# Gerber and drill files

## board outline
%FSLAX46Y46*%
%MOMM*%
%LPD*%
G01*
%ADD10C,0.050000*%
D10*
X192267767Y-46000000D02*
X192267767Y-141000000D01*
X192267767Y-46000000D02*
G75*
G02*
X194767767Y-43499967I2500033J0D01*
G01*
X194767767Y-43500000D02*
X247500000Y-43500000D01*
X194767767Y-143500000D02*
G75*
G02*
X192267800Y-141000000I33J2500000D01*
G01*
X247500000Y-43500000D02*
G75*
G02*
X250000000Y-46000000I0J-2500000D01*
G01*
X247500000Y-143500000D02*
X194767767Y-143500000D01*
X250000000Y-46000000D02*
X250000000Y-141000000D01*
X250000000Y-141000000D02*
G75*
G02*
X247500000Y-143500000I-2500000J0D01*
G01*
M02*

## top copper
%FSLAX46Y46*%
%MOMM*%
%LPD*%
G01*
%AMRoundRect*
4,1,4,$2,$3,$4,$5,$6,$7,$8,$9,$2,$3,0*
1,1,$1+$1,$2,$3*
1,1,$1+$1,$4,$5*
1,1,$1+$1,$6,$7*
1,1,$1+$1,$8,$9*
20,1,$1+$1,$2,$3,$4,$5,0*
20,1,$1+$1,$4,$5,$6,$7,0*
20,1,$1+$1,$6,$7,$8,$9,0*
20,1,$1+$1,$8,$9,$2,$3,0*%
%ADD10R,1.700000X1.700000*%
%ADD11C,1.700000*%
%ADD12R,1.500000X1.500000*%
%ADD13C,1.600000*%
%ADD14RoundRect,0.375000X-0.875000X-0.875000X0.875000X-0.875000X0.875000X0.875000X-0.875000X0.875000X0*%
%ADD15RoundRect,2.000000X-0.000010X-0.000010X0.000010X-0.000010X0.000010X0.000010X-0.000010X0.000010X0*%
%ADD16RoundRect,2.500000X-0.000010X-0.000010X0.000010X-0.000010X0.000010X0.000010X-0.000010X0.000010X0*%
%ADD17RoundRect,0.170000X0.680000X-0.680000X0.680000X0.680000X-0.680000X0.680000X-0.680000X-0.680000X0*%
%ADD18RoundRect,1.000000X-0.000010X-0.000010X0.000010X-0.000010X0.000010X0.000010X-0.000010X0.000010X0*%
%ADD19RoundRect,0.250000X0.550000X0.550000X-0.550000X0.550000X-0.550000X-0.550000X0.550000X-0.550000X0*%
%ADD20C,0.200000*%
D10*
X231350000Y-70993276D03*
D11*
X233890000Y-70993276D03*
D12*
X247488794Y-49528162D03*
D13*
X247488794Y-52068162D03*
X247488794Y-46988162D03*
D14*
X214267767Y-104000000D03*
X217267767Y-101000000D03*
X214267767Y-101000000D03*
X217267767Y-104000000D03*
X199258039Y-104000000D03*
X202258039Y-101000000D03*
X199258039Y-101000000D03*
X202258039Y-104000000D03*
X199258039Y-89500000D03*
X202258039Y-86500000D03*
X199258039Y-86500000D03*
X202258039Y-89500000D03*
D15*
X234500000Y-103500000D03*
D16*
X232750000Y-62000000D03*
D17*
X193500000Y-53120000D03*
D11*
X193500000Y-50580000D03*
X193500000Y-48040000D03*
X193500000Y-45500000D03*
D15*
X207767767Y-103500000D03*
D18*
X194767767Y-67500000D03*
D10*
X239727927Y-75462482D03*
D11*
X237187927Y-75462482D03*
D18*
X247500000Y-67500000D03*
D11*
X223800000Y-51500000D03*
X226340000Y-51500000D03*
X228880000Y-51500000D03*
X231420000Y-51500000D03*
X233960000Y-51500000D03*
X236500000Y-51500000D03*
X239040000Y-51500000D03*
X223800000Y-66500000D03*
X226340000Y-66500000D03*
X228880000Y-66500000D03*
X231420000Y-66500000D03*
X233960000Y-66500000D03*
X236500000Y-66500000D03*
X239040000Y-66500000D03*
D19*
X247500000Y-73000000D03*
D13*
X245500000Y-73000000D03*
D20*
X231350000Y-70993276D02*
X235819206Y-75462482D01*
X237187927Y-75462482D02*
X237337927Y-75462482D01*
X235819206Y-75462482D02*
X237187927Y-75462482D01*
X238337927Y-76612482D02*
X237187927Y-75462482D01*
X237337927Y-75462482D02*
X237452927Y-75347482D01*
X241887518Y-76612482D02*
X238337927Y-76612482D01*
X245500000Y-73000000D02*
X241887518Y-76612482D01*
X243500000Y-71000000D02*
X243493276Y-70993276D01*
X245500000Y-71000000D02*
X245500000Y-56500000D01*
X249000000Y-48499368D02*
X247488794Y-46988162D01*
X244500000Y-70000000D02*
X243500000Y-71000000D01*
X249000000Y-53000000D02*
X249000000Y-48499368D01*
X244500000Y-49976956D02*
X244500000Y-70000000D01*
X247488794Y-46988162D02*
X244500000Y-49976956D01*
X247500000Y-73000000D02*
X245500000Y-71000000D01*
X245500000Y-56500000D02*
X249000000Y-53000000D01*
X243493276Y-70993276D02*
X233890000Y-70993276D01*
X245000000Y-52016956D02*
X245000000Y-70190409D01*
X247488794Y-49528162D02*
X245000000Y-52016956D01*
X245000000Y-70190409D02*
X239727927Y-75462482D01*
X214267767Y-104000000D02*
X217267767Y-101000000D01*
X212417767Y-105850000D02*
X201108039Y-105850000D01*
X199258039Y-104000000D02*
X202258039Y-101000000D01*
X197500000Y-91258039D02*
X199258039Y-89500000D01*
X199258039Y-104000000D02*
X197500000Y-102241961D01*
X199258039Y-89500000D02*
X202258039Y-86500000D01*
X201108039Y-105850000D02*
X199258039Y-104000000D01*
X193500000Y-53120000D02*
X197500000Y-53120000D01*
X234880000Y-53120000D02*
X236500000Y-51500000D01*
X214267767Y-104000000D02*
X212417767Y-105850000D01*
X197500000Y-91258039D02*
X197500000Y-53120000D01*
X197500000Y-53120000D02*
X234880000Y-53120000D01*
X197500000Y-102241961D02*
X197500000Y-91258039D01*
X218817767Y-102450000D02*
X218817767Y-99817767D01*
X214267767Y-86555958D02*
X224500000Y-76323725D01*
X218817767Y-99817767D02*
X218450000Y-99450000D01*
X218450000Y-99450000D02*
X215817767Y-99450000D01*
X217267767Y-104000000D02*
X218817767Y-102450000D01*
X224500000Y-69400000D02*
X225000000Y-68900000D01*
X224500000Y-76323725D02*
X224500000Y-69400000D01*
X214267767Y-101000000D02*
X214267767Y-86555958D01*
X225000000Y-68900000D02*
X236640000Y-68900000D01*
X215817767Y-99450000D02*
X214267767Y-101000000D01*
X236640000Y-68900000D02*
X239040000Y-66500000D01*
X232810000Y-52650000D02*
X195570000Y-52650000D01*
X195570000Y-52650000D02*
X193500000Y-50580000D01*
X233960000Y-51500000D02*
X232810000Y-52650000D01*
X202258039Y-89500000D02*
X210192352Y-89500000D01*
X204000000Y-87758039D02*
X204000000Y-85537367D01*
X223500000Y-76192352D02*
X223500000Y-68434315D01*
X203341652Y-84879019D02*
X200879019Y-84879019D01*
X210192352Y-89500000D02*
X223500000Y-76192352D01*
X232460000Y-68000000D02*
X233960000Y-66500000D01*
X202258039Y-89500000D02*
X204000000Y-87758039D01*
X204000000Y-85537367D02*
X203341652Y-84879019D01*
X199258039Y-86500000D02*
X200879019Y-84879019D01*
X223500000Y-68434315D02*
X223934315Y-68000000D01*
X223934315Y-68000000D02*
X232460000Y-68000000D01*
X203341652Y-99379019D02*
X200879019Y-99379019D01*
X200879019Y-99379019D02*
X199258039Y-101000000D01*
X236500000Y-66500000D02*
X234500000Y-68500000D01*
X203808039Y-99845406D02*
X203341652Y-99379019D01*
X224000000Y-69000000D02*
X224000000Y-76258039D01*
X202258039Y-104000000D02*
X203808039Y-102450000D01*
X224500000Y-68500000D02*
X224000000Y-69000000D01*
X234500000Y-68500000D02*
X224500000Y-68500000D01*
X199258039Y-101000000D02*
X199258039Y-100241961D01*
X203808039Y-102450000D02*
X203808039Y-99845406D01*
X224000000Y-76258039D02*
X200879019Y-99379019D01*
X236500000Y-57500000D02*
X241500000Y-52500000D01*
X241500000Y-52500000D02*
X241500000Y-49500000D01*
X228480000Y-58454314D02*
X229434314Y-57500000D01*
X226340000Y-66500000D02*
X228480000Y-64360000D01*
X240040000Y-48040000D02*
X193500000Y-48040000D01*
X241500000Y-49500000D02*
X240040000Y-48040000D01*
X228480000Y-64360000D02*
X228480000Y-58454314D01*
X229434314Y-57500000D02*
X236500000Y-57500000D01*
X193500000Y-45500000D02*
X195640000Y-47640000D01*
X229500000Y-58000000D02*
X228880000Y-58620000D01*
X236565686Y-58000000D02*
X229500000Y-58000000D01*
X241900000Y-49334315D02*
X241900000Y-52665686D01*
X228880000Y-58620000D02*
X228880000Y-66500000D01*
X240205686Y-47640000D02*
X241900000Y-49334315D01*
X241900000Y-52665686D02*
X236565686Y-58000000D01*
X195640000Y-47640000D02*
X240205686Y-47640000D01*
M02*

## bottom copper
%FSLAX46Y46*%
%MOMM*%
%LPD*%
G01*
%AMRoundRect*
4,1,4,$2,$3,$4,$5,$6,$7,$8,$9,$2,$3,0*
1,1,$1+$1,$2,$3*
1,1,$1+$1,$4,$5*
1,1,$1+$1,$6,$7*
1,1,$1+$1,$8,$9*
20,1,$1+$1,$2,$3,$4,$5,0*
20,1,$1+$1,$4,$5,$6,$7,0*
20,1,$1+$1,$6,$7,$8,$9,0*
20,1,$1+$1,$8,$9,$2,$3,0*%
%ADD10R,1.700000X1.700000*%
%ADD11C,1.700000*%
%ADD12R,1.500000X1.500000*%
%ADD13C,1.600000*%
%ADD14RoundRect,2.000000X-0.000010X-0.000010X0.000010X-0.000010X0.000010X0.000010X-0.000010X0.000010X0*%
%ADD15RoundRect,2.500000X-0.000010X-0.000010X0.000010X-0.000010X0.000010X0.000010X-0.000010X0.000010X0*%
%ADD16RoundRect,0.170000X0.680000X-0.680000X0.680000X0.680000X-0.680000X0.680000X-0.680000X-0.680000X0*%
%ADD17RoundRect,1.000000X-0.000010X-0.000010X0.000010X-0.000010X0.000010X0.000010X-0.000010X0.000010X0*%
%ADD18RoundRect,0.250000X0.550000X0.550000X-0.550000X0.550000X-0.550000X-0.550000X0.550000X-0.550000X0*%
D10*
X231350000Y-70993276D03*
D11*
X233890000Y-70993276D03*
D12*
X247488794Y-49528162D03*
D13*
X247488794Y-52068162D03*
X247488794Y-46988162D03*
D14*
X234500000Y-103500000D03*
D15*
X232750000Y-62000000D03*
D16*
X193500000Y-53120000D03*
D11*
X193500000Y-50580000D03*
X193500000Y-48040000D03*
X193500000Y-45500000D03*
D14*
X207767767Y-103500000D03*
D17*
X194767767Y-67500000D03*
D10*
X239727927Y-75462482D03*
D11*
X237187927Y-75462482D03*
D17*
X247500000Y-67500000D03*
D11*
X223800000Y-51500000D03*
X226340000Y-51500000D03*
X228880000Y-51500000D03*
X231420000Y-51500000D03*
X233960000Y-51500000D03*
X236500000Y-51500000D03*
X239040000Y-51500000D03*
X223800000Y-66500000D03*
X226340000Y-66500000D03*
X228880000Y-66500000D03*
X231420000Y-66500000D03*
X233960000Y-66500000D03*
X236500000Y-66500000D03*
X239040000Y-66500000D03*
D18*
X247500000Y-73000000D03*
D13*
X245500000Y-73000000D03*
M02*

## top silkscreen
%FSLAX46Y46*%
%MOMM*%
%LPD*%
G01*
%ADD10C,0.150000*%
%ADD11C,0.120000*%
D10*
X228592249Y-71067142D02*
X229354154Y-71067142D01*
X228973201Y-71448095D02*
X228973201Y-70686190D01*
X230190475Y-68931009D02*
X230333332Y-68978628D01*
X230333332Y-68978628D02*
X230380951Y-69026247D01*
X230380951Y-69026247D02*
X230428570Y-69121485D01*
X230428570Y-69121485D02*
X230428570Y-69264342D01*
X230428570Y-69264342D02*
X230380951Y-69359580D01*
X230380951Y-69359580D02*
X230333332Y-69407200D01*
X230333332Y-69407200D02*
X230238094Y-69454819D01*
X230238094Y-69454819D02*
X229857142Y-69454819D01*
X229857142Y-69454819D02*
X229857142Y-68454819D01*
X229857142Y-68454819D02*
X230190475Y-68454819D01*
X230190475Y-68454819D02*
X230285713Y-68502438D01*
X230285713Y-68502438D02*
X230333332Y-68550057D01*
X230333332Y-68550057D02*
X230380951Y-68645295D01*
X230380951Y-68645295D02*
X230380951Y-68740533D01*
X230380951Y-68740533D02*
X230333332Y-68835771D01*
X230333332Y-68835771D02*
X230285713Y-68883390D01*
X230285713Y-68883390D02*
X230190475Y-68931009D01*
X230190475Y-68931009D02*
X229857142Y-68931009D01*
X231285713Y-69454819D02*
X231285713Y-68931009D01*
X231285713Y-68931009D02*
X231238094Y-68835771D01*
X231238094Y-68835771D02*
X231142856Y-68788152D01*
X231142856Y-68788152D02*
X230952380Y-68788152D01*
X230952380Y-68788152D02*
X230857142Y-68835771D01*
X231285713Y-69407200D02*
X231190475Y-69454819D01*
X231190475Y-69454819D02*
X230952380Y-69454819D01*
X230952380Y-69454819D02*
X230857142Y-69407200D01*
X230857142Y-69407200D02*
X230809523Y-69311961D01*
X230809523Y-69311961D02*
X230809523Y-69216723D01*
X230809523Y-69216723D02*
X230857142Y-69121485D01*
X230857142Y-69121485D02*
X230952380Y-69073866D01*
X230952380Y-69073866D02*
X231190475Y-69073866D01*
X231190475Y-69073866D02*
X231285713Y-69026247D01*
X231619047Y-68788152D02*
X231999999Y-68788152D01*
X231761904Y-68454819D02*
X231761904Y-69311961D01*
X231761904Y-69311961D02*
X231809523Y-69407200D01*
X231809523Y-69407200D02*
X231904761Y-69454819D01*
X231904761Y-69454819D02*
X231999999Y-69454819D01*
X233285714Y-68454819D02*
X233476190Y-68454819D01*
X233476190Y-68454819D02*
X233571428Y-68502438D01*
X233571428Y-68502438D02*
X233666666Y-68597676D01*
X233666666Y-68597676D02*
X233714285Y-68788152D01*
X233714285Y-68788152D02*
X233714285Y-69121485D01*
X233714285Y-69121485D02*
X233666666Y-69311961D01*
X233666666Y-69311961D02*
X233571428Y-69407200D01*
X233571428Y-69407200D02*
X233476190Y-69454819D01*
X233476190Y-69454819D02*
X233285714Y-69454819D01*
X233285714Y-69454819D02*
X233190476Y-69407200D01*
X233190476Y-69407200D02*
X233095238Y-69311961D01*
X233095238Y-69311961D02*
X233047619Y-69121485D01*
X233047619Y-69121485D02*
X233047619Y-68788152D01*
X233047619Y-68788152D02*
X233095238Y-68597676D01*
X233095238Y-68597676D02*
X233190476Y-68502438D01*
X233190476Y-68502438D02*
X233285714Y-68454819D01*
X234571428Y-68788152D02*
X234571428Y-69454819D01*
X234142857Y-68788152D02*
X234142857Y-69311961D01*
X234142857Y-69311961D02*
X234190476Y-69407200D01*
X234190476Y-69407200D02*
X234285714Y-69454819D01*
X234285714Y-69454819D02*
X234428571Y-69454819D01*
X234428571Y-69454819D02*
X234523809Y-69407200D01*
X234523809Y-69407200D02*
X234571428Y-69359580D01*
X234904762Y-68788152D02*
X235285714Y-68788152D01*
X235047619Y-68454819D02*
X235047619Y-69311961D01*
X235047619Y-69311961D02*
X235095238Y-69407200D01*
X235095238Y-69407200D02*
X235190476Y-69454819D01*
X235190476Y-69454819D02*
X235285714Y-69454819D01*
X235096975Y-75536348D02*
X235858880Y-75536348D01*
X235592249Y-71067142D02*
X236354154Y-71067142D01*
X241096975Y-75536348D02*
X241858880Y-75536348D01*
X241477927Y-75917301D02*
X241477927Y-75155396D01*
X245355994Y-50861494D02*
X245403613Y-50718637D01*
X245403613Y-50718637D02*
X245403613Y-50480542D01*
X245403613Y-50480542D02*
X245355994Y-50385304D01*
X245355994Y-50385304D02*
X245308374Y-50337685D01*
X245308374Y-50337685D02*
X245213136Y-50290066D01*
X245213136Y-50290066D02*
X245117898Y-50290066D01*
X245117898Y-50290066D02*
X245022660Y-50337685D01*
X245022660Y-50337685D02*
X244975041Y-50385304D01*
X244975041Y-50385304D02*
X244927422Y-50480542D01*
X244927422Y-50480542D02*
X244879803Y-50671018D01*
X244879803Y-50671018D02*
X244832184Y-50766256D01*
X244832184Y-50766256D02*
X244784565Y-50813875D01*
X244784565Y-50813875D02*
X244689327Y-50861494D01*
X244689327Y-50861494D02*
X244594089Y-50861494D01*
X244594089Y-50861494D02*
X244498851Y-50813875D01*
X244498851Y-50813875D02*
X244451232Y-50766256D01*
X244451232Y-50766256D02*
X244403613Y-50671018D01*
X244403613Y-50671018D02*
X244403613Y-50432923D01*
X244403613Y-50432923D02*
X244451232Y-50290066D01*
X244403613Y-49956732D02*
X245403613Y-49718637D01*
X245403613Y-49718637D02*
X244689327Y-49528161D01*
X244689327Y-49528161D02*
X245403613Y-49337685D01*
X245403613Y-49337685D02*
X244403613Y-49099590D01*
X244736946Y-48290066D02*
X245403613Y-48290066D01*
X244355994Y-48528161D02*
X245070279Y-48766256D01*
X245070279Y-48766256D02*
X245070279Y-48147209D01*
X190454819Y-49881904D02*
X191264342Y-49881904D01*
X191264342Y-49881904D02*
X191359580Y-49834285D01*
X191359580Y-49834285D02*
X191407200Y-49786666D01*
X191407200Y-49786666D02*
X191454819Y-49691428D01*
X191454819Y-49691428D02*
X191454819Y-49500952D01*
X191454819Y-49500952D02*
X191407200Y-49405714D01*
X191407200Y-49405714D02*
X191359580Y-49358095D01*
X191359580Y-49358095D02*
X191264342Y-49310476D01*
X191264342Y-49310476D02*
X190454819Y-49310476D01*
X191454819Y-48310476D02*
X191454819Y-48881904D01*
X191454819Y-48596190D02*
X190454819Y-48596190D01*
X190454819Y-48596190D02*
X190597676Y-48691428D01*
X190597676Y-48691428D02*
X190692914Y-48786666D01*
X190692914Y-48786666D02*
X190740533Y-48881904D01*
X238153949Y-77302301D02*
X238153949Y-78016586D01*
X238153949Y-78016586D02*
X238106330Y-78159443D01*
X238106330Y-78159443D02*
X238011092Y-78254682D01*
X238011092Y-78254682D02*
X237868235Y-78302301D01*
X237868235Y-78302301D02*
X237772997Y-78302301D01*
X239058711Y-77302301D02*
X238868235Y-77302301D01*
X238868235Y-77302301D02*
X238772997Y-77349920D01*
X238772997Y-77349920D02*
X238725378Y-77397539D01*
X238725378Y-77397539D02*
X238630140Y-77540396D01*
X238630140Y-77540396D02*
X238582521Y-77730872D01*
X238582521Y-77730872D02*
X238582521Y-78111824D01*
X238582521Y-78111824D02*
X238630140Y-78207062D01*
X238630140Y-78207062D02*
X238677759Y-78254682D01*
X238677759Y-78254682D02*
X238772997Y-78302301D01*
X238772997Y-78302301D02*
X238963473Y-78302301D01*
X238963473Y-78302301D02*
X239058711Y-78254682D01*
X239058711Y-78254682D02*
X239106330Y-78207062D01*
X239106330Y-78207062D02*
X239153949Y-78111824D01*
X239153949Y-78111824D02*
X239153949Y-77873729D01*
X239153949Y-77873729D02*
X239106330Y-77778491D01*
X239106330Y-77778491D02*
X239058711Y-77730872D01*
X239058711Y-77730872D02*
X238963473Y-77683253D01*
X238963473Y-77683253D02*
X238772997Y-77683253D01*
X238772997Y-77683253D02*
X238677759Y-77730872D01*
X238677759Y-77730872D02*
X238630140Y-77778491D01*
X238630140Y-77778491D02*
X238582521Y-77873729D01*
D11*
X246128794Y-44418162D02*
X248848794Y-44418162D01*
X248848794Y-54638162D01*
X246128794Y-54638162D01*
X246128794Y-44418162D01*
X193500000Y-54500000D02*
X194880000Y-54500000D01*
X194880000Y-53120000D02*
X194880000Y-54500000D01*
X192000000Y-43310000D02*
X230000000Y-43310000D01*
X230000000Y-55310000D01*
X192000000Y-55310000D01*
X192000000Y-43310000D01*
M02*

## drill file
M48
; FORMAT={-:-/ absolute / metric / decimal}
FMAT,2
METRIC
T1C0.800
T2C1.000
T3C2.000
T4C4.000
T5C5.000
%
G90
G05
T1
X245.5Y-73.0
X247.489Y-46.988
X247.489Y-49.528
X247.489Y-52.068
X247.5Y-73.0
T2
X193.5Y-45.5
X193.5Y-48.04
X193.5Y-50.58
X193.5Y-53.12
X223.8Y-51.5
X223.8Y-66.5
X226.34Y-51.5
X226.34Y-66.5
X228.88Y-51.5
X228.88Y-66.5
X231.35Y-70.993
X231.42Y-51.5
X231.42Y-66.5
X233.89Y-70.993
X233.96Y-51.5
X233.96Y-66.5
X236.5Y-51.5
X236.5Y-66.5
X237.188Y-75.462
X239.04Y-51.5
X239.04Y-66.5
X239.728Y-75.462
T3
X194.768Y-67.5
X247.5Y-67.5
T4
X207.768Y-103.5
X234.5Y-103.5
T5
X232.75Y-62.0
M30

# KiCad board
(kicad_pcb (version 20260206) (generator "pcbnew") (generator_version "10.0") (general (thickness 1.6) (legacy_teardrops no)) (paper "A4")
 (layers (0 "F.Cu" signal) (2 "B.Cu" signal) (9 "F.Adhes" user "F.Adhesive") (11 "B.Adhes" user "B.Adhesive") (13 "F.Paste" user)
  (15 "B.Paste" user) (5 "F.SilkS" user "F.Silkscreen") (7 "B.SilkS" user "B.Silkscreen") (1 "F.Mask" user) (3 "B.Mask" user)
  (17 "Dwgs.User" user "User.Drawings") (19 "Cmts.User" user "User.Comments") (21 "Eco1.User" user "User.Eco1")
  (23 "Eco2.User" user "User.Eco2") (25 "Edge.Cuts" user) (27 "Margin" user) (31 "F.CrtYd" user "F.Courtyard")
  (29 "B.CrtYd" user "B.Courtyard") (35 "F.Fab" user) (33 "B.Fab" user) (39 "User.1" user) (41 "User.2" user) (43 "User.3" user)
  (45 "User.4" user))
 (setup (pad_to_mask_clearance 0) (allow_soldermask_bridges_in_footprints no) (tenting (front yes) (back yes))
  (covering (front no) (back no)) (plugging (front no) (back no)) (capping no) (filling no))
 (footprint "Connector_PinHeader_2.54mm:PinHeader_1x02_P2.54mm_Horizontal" (layer "F.Cu") (at 231.35 70.993276 90)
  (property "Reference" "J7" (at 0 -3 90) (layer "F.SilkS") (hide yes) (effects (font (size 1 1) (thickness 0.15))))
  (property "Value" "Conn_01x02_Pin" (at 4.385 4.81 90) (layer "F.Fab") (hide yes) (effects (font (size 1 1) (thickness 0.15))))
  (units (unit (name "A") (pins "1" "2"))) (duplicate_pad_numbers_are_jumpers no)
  (pad "1" thru_hole rect (at 0 0 90) (size 1.7 1.7) (drill 1) (layers "*.Cu" "*.Mask") (remove_unused_layers no) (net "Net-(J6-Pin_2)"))
  (pad "2" thru_hole circle (at 0 2.54 90) (size 1.7 1.7) (drill 1) (layers "*.Cu" "*.Mask") (remove_unused_layers no)
   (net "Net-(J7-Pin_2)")))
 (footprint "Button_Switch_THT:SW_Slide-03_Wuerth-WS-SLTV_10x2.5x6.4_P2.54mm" (layer "F.Cu") (at 247.488794 49.528162 90)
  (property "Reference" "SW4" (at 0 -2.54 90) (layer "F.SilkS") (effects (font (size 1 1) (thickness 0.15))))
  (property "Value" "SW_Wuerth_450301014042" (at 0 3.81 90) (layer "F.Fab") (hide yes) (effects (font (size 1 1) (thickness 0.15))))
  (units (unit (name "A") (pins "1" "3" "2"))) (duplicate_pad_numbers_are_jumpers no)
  (fp_rect (start -5.11 -1.36) (end 5.11 1.36) (stroke (width 0.12) (type default)) (fill no) (layer "F.SilkS"))
  (pad "1" thru_hole rect (at 0 0 90) (size 1.5 1.5) (drill 0.8) (layers "*.Cu" "*.Mask") (remove_unused_layers no) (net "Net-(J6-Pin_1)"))
  (pad "2" thru_hole circle (at -2.54 0 90) (size 1.6 1.6) (drill 0.8) (layers "*.Cu" "*.Mask") (remove_unused_layers no)
   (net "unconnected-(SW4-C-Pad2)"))
  (pad "3" thru_hole circle (at 2.54 0 90) (size 1.6 1.6) (drill 0.8) (layers "*.Cu" "*.Mask") (remove_unused_layers no)
   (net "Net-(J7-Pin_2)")))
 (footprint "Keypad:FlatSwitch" (layer "F.Cu") (at 215.767767 102.5)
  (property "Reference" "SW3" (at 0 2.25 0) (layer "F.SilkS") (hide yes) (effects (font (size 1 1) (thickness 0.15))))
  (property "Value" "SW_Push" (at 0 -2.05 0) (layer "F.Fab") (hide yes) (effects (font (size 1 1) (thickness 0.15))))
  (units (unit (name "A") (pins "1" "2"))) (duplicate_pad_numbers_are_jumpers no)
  (pad "1" smd roundrect (at -1.5 1.5) (size 2.5 2.5) (layers "*.Mask" "F.Cu") (roundrect_rratio 0.15) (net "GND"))
  (pad "1" smd roundrect (at 1.5 -1.5) (size 2.5 2.5) (layers "*.Mask" "F.Cu") (roundrect_rratio 0.15) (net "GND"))
  (pad "2" smd roundrect (at -1.5 -1.5) (size 2.5 2.5) (layers "*.Mask" "F.Cu") (roundrect_rratio 0.15) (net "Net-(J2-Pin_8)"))
  (pad "2" smd roundrect (at 1.5 1.5) (size 2.5 2.5) (layers "*.Mask" "F.Cu") (roundrect_rratio 0.15) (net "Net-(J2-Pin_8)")))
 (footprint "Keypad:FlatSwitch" (layer "F.Cu") (at 200.758039 102.5)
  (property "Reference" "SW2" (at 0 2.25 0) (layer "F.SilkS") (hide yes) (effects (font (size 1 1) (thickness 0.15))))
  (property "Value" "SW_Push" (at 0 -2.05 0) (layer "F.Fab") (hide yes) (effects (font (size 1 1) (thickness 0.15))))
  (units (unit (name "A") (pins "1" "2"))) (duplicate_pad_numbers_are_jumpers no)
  (pad "1" smd roundrect (at -1.5 1.5) (size 2.5 2.5) (layers "*.Mask" "F.Cu") (roundrect_rratio 0.15) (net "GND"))
  (pad "1" smd roundrect (at 1.5 -1.5) (size 2.5 2.5) (layers "*.Mask" "F.Cu") (roundrect_rratio 0.15) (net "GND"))
  (pad "2" smd roundrect (at -1.5 -1.5) (size 2.5 2.5) (layers "*.Mask" "F.Cu") (roundrect_rratio 0.15) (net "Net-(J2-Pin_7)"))
  (pad "2" smd roundrect (at 1.5 1.5) (size 2.5 2.5) (layers "*.Mask" "F.Cu") (roundrect_rratio 0.15) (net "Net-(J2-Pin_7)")))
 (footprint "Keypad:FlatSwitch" (layer "F.Cu") (at 200.758039 88)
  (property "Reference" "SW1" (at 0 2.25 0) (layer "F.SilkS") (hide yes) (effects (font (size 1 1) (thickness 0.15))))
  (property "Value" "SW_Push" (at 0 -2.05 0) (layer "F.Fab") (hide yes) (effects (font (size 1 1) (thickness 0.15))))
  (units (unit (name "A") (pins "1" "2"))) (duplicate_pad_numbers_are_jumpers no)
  (pad "1" smd roundrect (at -1.5 1.5) (size 2.5 2.5) (layers "*.Mask" "F.Cu") (roundrect_rratio 0.15) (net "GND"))
  (pad "1" smd roundrect (at 1.5 -1.5) (size 2.5 2.5) (layers "*.Mask" "F.Cu") (roundrect_rratio 0.15) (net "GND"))
  (pad "2" smd roundrect (at -1.5 -1.5) (size 2.5 2.5) (layers "*.Mask" "F.Cu") (roundrect_rratio 0.15) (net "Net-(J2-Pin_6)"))
  (pad "2" smd roundrect (at 1.5 1.5) (size 2.5 2.5) (layers "*.Mask" "F.Cu") (roundrect_rratio 0.15) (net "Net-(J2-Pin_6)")))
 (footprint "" (layer "F.Cu") (at 234.5 103.5)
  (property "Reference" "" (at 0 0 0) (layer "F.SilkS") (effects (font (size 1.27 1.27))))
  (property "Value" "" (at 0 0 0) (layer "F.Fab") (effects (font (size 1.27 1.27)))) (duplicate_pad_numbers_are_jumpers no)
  (pad "" np_thru_hole roundrect (at 0 0) (size 4 4) (drill 4) (layers "*.Cu" "*.Mask") (roundrect_rratio 0.5)))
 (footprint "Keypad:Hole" (layer "F.Cu") (at 232.75 62)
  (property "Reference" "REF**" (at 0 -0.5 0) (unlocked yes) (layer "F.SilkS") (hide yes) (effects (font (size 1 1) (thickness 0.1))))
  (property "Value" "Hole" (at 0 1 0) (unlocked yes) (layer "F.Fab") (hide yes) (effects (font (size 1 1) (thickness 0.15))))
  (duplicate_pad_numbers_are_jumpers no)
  (pad "" np_thru_hole roundrect (at 0 0) (size 5 5) (drill 5) (layers "*.Cu" "*.Mask") (roundrect_rratio 0.5)))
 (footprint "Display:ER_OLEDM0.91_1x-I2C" (layer "F.Cu") (at 193.5 53.12 90)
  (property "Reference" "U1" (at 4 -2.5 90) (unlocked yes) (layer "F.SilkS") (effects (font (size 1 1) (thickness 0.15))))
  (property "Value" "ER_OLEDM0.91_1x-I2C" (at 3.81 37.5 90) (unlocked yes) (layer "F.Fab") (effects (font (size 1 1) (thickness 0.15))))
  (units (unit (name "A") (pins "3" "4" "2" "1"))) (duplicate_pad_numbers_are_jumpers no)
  (fp_line (start -1.38 0) (end -1.38 1.38) (stroke (width 0.12) (type solid)) (layer "F.SilkS"))
  (fp_line (start 0 1.38) (end -1.38 1.38) (stroke (width 0.12) (type solid)) (layer "F.SilkS"))
  (fp_rect (start -2.19 -1.5) (end 9.81 36.5) (stroke (width 0.12) (type solid)) (fill no) (layer "F.SilkS"))
  (pad "1" thru_hole roundrect (at 0 0 90) (size 1.7 1.7) (drill 1) (layers "*.Cu" "*.Mask") (remove_unused_layers no)
   (roundrect_rratio 0.1) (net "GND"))
  (pad "2" thru_hole circle (at 2.54 0 90) (size 1.7 1.7) (drill 1) (layers "*.Cu" "*.Mask") (remove_unused_layers no)
   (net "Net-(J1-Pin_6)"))
  (pad "3" thru_hole circle (at 5.08 0 90) (size 1.7 1.7) (drill 1) (layers "*.Cu" "*.Mask") (remove_unused_layers no)
   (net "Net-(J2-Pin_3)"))
  (pad "4" thru_hole circle (at 7.62 0 90) (size 1.7 1.7) (drill 1) (layers "*.Cu" "*.Mask") (remove_unused_layers no)
   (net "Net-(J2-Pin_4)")))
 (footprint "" (layer "F.Cu") (at 207.767767 103.5)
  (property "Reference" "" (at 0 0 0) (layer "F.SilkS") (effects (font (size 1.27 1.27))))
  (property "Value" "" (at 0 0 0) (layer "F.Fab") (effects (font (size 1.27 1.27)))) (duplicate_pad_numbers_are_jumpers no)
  (pad "" np_thru_hole roundrect (at 0 0) (size 4 4) (drill 4) (layers "*.Cu" "*.Mask") (roundrect_rratio 0.5)))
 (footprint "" (layer "F.Cu") (at 194.767767 67.5)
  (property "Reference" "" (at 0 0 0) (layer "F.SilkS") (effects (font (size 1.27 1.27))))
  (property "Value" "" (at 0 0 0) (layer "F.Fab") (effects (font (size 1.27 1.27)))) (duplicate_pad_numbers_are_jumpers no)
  (pad "" np_thru_hole roundrect (at 0 0) (size 2 2) (drill 2) (layers "*.Cu" "*.Mask") (roundrect_rratio 0.5)))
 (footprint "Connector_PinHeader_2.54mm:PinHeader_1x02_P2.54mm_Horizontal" (layer "F.Cu") (at 239.727927 75.462482 -90)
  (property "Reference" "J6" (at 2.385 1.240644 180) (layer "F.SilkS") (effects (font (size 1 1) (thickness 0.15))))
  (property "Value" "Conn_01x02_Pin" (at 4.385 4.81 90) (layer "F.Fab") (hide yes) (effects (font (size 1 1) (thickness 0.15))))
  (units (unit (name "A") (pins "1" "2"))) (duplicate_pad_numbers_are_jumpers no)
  (pad "1" thru_hole rect (at 0 0 270) (size 1.7 1.7) (drill 1) (layers "*.Cu" "*.Mask") (remove_unused_layers no) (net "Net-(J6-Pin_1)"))
  (pad "2" thru_hole circle (at 0 2.54 270) (size 1.7 1.7) (drill 1) (layers "*.Cu" "*.Mask") (remove_unused_layers no)
   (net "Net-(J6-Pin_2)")))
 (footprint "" (layer "F.Cu") (at 247.5 67.5)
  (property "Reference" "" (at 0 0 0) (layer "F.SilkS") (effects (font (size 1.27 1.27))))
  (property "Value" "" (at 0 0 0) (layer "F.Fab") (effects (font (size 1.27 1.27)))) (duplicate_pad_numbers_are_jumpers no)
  (pad "" np_thru_hole roundrect (at 0 0) (size 2 2) (drill 2) (layers "*.Cu" "*.Mask") (roundrect_rratio 0.5)))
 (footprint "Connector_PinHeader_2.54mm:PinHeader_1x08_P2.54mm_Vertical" (layer "B.Cu") (at 221.26 51.5 -90)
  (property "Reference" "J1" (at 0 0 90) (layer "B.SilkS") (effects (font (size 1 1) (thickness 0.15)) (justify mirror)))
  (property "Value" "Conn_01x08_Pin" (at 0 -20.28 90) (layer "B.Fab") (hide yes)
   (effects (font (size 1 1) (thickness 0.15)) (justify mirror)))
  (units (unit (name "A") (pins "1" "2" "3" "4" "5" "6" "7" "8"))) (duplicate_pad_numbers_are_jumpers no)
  (pad "2" thru_hole circle (at 0 -2.54 270) (size 1.7 1.7) (drill 1) (layers "*.Cu" "*.Mask") (remove_unused_layers no)
   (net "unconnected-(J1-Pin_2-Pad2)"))
  (pad "3" thru_hole circle (at 0 -5.08 270) (size 1.7 1.7) (drill 1) (layers "*.Cu" "*.Mask") (remove_unused_layers no)
   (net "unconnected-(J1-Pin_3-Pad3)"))
  (pad "4" thru_hole circle (at 0 -7.62 270) (size 1.7 1.7) (drill 1) (layers "*.Cu" "*.Mask") (remove_unused_layers no)
   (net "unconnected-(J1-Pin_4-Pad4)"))
  (pad "5" thru_hole circle (at 0 -10.16 270) (size 1.7 1.7) (drill 1) (layers "*.Cu" "*.Mask") (remove_unused_layers no)
   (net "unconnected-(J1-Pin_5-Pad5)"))
  (pad "6" thru_hole circle (at 0 -12.7 270) (size 1.7 1.7) (drill 1) (layers "*.Cu" "*.Mask") (remove_unused_layers no)
   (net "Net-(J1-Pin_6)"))
  (pad "7" thru_hole circle (at 0 -15.24 270) (size 1.7 1.7) (drill 1) (layers "*.Cu" "*.Mask") (remove_unused_layers no) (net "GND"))
  (pad "8" thru_hole circle (at 0 -17.78 270) (size 1.7 1.7) (drill 1) (layers "*.Cu" "*.Mask") (remove_unused_layers no)
   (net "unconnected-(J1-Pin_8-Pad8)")))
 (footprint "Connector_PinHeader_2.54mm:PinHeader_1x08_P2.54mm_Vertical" (layer "B.Cu") (at 221.26 66.5 -90)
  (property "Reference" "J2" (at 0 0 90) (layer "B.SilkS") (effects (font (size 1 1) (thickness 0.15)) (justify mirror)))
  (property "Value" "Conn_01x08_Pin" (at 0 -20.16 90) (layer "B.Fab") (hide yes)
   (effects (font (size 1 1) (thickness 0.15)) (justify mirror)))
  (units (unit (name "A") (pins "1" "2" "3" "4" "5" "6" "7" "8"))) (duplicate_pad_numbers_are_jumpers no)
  (pad "2" thru_hole circle (at 0 -2.54 270) (size 1.7 1.7) (drill 1) (layers "*.Cu" "*.Mask") (remove_unused_layers no)
   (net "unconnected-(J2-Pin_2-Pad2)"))
  (pad "3" thru_hole circle (at 0 -5.08 270) (size 1.7 1.7) (drill 1) (layers "*.Cu" "*.Mask") (remove_unused_layers no)
   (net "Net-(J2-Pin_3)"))
  (pad "4" thru_hole circle (at 0 -7.62 270) (size 1.7 1.7) (drill 1) (layers "*.Cu" "*.Mask") (remove_unused_layers no)
   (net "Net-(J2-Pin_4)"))
  (pad "5" thru_hole circle (at 0 -10.16 270) (size 1.7 1.7) (drill 1) (layers "*.Cu" "*.Mask") (remove_unused_layers no)
   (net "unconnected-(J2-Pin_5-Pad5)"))
  (pad "6" thru_hole circle (at 0 -12.7 270) (size 1.7 1.7) (drill 1) (layers "*.Cu" "*.Mask") (remove_unused_layers no)
   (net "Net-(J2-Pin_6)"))
  (pad "7" thru_hole circle (at 0 -15.24 270) (size 1.7 1.7) (drill 1) (layers "*.Cu" "*.Mask") (remove_unused_layers no)
   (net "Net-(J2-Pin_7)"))
  (pad "8" thru_hole circle (at 0 -17.78 270) (size 1.7 1.7) (drill 1) (layers "*.Cu" "*.Mask") (remove_unused_layers no)
   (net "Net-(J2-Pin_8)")))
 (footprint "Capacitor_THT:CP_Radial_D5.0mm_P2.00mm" (layer "B.Cu") (at 247.5 73 180)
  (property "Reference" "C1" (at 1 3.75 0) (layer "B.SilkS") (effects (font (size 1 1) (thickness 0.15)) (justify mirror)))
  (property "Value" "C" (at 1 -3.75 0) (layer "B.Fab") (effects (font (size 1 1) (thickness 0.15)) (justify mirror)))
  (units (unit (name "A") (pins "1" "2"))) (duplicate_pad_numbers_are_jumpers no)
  (pad "1" thru_hole roundrect (at 0 0 180) (size 1.6 1.6) (drill 0.8) (layers "*.Cu" "*.Mask") (remove_unused_layers no)
   (roundrect_rratio 0.15625) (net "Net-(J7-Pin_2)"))
  (pad "2" thru_hole circle (at 2 0 180) (size 1.6 1.6) (drill 0.8) (layers "*.Cu" "*.Mask") (remove_unused_layers no)
   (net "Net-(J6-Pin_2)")))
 (gr_line (start 192.267767 46) (end 192.267767 141) (stroke (width 0.05) (type default)) (layer "Edge.Cuts"))
 (gr_arc (start 192.267767 46) (mid 193 44.232233) (end 194.767767 43.5) (stroke (width 0.05) (type default)) (layer "Edge.Cuts"))
 (gr_line (start 194.767767 43.5) (end 247.5 43.5) (stroke (width 0.05) (type default)) (layer "Edge.Cuts"))
 (gr_arc (start 194.767767 143.5) (mid 193 142.767767) (end 192.267767 141) (stroke (width 0.05) (type default)) (layer "Edge.Cuts"))
 (gr_arc (start 247.5 43.5) (mid 249.267767 44.232233) (end 250 46) (stroke (width 0.05) (type default)) (layer "Edge.Cuts"))
 (gr_line (start 247.5 143.5) (end 194.767767 143.5) (stroke (width 0.05) (type default)) (layer "Edge.Cuts"))
 (gr_line (start 250 46) (end 250 141) (stroke (width 0.05) (type default)) (layer "Edge.Cuts"))
 (gr_arc (start 250 141) (mid 249.267767 142.767767) (end 247.5 143.5) (stroke (width 0.05) (type default)) (layer "Edge.Cuts"))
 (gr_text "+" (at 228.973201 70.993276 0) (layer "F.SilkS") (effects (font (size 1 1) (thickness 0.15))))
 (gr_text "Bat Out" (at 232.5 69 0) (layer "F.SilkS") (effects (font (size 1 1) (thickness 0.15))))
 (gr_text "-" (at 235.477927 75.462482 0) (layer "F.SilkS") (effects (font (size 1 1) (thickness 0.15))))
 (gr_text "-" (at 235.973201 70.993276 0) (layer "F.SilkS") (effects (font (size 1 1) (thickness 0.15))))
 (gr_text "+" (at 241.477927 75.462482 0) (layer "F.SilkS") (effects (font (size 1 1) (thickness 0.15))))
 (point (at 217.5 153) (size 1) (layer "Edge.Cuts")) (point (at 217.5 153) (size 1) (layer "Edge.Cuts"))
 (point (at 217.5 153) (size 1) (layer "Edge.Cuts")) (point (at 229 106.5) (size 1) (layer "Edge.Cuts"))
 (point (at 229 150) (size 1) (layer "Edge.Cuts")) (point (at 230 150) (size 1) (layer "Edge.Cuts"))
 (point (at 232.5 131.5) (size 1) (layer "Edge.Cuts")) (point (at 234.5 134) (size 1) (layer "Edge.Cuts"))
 (segment (start 231.35 70.993276) (end 235.819206 75.462482) (width 0.2) (layer "F.Cu") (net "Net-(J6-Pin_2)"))
 (segment (start 237.187927 75.462482) (end 237.337927 75.462482) (width 0.2) (layer "F.Cu") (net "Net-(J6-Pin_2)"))
 (segment (start 235.819206 75.462482) (end 237.187927 75.462482) (width 0.2) (layer "F.Cu") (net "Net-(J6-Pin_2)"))
 (segment (start 238.337927 76.612482) (end 237.187927 75.462482) (width 0.2) (layer "F.Cu") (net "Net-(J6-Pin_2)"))
 (segment (start 237.337927 75.462482) (end 237.452927 75.347482) (width 0.2) (layer "F.Cu") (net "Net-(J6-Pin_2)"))
 (segment (start 241.887518 76.612482) (end 238.337927 76.612482) (width 0.2) (layer "F.Cu") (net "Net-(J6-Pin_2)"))
 (segment (start 245.5 73) (end 241.887518 76.612482) (width 0.2) (layer "F.Cu") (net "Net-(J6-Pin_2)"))
 (segment (start 243.5 71) (end 243.493276 70.993276) (width 0.2) (layer "F.Cu") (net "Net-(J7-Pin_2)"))
 (segment (start 245.5 71) (end 245.5 56.5) (width 0.2) (layer "F.Cu") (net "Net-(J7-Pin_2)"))
 (segment (start 249 48.499368) (end 247.488794 46.988162) (width 0.2) (layer "F.Cu") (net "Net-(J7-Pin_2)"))
 (segment (start 244.5 70) (end 243.5 71) (width 0.2) (layer "F.Cu") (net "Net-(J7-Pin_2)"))
 (segment (start 249 53) (end 249 48.499368) (width 0.2) (layer "F.Cu") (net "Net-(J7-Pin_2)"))
 (segment (start 244.5 49.976956) (end 244.5 70) (width 0.2) (layer "F.Cu") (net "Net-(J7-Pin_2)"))
 (segment (start 247.488794 46.988162) (end 244.5 49.976956) (width 0.2) (layer "F.Cu") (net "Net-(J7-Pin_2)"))
 (segment (start 247.5 73) (end 245.5 71) (width 0.2) (layer "F.Cu") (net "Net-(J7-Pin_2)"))
 (segment (start 245.5 56.5) (end 249 53) (width 0.2) (layer "F.Cu") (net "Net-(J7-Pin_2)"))
 (segment (start 243.493276 70.993276) (end 233.89 70.993276) (width 0.2) (layer "F.Cu") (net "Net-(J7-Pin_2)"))
 (segment (start 245 52.016956) (end 245 70.190409) (width 0.2) (layer "F.Cu") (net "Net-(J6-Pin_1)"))
 (segment (start 247.488794 49.528162) (end 245 52.016956) (width 0.2) (layer "F.Cu") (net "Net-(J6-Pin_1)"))
 (segment (start 245 70.190409) (end 239.727927 75.462482) (width 0.2) (layer "F.Cu") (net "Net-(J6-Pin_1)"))
 (segment (start 214.267767 104) (end 217.267767 101) (width 0.2) (layer "F.Cu") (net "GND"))
 (segment (start 212.417767 105.85) (end 201.108039 105.85) (width 0.2) (layer "F.Cu") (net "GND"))
 (segment (start 199.258039 104) (end 202.258039 101) (width 0.2) (layer "F.Cu") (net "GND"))
 (segment (start 197.5 91.258039) (end 199.258039 89.5) (width 0.2) (layer "F.Cu") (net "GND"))
 (segment (start 199.258039 104) (end 197.5 102.241961) (width 0.2) (layer "F.Cu") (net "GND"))
 (segment (start 199.258039 89.5) (end 202.258039 86.5) (width 0.2) (layer "F.Cu") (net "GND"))
 (segment (start 201.108039 105.85) (end 199.258039 104) (width 0.2) (layer "F.Cu") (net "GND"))
 (segment (start 193.5 53.12) (end 197.5 53.12) (width 0.2) (layer "F.Cu") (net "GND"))
 (segment (start 234.88 53.12) (end 236.5 51.5) (width 0.2) (layer "F.Cu") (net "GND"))
 (segment (start 214.267767 104) (end 212.417767 105.85) (width 0.2) (layer "F.Cu") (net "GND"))
 (segment (start 197.5 91.258039) (end 197.5 53.12) (width 0.2) (layer "F.Cu") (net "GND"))
 (segment (start 197.5 53.12) (end 234.88 53.12) (width 0.2) (layer "F.Cu") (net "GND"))
 (segment (start 197.5 102.241961) (end 197.5 91.258039) (width 0.2) (layer "F.Cu") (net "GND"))
 (segment (start 218.817767 102.45) (end 218.817767 99.817767) (width 0.2) (layer "F.Cu") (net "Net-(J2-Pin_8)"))
 (segment (start 214.267767 86.555958) (end 224.5 76.323725) (width 0.2) (layer "F.Cu") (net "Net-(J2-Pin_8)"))
 (segment (start 218.817767 99.817767) (end 218.45 99.45) (width 0.2) (layer "F.Cu") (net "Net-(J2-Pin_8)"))
 (segment (start 218.45 99.45) (end 215.817767 99.45) (width 0.2) (layer "F.Cu") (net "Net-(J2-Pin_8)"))
 (segment (start 217.267767 104) (end 218.817767 102.45) (width 0.2) (layer "F.Cu") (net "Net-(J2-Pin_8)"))
 (segment (start 224.5 69.4) (end 225 68.9) (width 0.2) (layer "F.Cu") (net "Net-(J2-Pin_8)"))
 (segment (start 224.5 76.323725) (end 224.5 69.4) (width 0.2) (layer "F.Cu") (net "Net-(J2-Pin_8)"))
 (segment (start 214.267767 101) (end 214.267767 86.555958) (width 0.2) (layer "F.Cu") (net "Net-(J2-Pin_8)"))
 (segment (start 225 68.9) (end 236.64 68.9) (width 0.2) (layer "F.Cu") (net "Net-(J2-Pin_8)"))
 (segment (start 215.817767 99.45) (end 214.267767 101) (width 0.2) (layer "F.Cu") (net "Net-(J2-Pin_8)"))
 (segment (start 236.64 68.9) (end 239.04 66.5) (width 0.2) (layer "F.Cu") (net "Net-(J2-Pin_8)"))
 (segment (start 232.81 52.65) (end 195.57 52.65) (width 0.2) (layer "F.Cu") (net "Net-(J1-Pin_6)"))
 (segment (start 195.57 52.65) (end 193.5 50.58) (width 0.2) (layer "F.Cu") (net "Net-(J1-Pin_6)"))
 (segment (start 233.96 51.5) (end 232.81 52.65) (width 0.2) (layer "F.Cu") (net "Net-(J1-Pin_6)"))
 (segment (start 202.258039 89.5) (end 210.192352 89.5) (width 0.2) (layer "F.Cu") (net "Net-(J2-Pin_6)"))
 (segment (start 204 87.758039) (end 204 85.537367) (width 0.2) (layer "F.Cu") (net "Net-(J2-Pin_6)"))
 (segment (start 223.5 76.192352) (end 223.5 68.434315) (width 0.2) (layer "F.Cu") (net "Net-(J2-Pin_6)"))
 (segment (start 203.341652 84.879019) (end 200.879019 84.879019) (width 0.2) (layer "F.Cu") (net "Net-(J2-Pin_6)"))
 (segment (start 210.192352 89.5) (end 223.5 76.192352) (width 0.2) (layer "F.Cu") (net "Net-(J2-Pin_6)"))
 (segment (start 232.46 68) (end 233.96 66.5) (width 0.2) (layer "F.Cu") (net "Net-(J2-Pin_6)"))
 (segment (start 202.258039 89.5) (end 204 87.758039) (width 0.2) (layer "F.Cu") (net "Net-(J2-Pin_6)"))
 (segment (start 204 85.537367) (end 203.341652 84.879019) (width 0.2) (layer "F.Cu") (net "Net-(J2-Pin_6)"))
 (segment (start 199.258039 86.5) (end 200.879019 84.879019) (width 0.2) (layer "F.Cu") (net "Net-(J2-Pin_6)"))
 (segment (start 223.5 68.434315) (end 223.934315 68) (width 0.2) (layer "F.Cu") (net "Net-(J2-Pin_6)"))
 (segment (start 223.934315 68) (end 232.46 68) (width 0.2) (layer "F.Cu") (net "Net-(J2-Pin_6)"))
 (segment (start 203.341652 99.379019) (end 200.879019 99.379019) (width 0.2) (layer "F.Cu") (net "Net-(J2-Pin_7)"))
 (segment (start 200.879019 99.379019) (end 199.258039 101) (width 0.2) (layer "F.Cu") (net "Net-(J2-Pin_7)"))
 (segment (start 236.5 66.5) (end 234.5 68.5) (width 0.2) (layer "F.Cu") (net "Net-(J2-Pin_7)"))
 (segment (start 203.808039 99.845406) (end 203.341652 99.379019) (width 0.2) (layer "F.Cu") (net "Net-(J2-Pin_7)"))
 (segment (start 224 69) (end 224 76.258039) (width 0.2) (layer "F.Cu") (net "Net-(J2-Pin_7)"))
 (segment (start 202.258039 104) (end 203.808039 102.45) (width 0.2) (layer "F.Cu") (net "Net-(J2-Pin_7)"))
 (segment (start 224.5 68.5) (end 224 69) (width 0.2) (layer "F.Cu") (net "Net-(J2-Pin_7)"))
 (segment (start 234.5 68.5) (end 224.5 68.5) (width 0.2) (layer "F.Cu") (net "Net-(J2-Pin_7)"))
 (segment (start 199.258039 101) (end 199.258039 100.241961) (width 0.2) (layer "F.Cu") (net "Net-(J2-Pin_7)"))
 (segment (start 203.808039 102.45) (end 203.808039 99.845406) (width 0.2) (layer "F.Cu") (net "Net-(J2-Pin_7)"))
 (segment (start 224 76.258039) (end 200.879019 99.379019) (width 0.2) (layer "F.Cu") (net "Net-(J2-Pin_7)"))
 (segment (start 236.5 57.5) (end 241.5 52.5) (width 0.2) (layer "F.Cu") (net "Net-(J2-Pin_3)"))
 (segment (start 241.5 52.5) (end 241.5 49.5) (width 0.2) (layer "F.Cu") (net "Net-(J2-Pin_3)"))
 (segment (start 228.48 58.454314) (end 229.434314 57.5) (width 0.2) (layer "F.Cu") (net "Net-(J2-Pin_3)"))
 (segment (start 226.34 66.5) (end 228.48 64.36) (width 0.2) (layer "F.Cu") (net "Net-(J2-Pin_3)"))
 (segment (start 240.04 48.04) (end 193.5 48.04) (width 0.2) (layer "F.Cu") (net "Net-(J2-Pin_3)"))
 (segment (start 241.5 49.5) (end 240.04 48.04) (width 0.2) (layer "F.Cu") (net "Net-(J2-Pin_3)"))
 (segment (start 228.48 64.36) (end 228.48 58.454314) (width 0.2) (layer "F.Cu") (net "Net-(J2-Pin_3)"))
 (segment (start 229.434314 57.5) (end 236.5 57.5) (width 0.2) (layer "F.Cu") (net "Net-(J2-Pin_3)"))
 (segment (start 193.5 45.5) (end 195.64 47.64) (width 0.2) (layer "F.Cu") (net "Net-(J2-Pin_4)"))
 (segment (start 229.5 58) (end 228.88 58.62) (width 0.2) (layer "F.Cu") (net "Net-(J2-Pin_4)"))
 (segment (start 236.565686 58) (end 229.5 58) (width 0.2) (layer "F.Cu") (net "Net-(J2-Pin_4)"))
 (segment (start 241.9 49.334315) (end 241.9 52.665686) (width 0.2) (layer "F.Cu") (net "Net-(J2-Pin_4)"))
 (segment (start 228.88 58.62) (end 228.88 66.5) (width 0.2) (layer "F.Cu") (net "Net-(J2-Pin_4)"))
 (segment (start 240.205686 47.64) (end 241.9 49.334315) (width 0.2) (layer "F.Cu") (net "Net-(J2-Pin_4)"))
 (segment (start 241.9 52.665686) (end 236.565686 58) (width 0.2) (layer "F.Cu") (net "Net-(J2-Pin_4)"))
 (segment (start 195.64 47.64) (end 240.205686 47.64) (width 0.2) (layer "F.Cu") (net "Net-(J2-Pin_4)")))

